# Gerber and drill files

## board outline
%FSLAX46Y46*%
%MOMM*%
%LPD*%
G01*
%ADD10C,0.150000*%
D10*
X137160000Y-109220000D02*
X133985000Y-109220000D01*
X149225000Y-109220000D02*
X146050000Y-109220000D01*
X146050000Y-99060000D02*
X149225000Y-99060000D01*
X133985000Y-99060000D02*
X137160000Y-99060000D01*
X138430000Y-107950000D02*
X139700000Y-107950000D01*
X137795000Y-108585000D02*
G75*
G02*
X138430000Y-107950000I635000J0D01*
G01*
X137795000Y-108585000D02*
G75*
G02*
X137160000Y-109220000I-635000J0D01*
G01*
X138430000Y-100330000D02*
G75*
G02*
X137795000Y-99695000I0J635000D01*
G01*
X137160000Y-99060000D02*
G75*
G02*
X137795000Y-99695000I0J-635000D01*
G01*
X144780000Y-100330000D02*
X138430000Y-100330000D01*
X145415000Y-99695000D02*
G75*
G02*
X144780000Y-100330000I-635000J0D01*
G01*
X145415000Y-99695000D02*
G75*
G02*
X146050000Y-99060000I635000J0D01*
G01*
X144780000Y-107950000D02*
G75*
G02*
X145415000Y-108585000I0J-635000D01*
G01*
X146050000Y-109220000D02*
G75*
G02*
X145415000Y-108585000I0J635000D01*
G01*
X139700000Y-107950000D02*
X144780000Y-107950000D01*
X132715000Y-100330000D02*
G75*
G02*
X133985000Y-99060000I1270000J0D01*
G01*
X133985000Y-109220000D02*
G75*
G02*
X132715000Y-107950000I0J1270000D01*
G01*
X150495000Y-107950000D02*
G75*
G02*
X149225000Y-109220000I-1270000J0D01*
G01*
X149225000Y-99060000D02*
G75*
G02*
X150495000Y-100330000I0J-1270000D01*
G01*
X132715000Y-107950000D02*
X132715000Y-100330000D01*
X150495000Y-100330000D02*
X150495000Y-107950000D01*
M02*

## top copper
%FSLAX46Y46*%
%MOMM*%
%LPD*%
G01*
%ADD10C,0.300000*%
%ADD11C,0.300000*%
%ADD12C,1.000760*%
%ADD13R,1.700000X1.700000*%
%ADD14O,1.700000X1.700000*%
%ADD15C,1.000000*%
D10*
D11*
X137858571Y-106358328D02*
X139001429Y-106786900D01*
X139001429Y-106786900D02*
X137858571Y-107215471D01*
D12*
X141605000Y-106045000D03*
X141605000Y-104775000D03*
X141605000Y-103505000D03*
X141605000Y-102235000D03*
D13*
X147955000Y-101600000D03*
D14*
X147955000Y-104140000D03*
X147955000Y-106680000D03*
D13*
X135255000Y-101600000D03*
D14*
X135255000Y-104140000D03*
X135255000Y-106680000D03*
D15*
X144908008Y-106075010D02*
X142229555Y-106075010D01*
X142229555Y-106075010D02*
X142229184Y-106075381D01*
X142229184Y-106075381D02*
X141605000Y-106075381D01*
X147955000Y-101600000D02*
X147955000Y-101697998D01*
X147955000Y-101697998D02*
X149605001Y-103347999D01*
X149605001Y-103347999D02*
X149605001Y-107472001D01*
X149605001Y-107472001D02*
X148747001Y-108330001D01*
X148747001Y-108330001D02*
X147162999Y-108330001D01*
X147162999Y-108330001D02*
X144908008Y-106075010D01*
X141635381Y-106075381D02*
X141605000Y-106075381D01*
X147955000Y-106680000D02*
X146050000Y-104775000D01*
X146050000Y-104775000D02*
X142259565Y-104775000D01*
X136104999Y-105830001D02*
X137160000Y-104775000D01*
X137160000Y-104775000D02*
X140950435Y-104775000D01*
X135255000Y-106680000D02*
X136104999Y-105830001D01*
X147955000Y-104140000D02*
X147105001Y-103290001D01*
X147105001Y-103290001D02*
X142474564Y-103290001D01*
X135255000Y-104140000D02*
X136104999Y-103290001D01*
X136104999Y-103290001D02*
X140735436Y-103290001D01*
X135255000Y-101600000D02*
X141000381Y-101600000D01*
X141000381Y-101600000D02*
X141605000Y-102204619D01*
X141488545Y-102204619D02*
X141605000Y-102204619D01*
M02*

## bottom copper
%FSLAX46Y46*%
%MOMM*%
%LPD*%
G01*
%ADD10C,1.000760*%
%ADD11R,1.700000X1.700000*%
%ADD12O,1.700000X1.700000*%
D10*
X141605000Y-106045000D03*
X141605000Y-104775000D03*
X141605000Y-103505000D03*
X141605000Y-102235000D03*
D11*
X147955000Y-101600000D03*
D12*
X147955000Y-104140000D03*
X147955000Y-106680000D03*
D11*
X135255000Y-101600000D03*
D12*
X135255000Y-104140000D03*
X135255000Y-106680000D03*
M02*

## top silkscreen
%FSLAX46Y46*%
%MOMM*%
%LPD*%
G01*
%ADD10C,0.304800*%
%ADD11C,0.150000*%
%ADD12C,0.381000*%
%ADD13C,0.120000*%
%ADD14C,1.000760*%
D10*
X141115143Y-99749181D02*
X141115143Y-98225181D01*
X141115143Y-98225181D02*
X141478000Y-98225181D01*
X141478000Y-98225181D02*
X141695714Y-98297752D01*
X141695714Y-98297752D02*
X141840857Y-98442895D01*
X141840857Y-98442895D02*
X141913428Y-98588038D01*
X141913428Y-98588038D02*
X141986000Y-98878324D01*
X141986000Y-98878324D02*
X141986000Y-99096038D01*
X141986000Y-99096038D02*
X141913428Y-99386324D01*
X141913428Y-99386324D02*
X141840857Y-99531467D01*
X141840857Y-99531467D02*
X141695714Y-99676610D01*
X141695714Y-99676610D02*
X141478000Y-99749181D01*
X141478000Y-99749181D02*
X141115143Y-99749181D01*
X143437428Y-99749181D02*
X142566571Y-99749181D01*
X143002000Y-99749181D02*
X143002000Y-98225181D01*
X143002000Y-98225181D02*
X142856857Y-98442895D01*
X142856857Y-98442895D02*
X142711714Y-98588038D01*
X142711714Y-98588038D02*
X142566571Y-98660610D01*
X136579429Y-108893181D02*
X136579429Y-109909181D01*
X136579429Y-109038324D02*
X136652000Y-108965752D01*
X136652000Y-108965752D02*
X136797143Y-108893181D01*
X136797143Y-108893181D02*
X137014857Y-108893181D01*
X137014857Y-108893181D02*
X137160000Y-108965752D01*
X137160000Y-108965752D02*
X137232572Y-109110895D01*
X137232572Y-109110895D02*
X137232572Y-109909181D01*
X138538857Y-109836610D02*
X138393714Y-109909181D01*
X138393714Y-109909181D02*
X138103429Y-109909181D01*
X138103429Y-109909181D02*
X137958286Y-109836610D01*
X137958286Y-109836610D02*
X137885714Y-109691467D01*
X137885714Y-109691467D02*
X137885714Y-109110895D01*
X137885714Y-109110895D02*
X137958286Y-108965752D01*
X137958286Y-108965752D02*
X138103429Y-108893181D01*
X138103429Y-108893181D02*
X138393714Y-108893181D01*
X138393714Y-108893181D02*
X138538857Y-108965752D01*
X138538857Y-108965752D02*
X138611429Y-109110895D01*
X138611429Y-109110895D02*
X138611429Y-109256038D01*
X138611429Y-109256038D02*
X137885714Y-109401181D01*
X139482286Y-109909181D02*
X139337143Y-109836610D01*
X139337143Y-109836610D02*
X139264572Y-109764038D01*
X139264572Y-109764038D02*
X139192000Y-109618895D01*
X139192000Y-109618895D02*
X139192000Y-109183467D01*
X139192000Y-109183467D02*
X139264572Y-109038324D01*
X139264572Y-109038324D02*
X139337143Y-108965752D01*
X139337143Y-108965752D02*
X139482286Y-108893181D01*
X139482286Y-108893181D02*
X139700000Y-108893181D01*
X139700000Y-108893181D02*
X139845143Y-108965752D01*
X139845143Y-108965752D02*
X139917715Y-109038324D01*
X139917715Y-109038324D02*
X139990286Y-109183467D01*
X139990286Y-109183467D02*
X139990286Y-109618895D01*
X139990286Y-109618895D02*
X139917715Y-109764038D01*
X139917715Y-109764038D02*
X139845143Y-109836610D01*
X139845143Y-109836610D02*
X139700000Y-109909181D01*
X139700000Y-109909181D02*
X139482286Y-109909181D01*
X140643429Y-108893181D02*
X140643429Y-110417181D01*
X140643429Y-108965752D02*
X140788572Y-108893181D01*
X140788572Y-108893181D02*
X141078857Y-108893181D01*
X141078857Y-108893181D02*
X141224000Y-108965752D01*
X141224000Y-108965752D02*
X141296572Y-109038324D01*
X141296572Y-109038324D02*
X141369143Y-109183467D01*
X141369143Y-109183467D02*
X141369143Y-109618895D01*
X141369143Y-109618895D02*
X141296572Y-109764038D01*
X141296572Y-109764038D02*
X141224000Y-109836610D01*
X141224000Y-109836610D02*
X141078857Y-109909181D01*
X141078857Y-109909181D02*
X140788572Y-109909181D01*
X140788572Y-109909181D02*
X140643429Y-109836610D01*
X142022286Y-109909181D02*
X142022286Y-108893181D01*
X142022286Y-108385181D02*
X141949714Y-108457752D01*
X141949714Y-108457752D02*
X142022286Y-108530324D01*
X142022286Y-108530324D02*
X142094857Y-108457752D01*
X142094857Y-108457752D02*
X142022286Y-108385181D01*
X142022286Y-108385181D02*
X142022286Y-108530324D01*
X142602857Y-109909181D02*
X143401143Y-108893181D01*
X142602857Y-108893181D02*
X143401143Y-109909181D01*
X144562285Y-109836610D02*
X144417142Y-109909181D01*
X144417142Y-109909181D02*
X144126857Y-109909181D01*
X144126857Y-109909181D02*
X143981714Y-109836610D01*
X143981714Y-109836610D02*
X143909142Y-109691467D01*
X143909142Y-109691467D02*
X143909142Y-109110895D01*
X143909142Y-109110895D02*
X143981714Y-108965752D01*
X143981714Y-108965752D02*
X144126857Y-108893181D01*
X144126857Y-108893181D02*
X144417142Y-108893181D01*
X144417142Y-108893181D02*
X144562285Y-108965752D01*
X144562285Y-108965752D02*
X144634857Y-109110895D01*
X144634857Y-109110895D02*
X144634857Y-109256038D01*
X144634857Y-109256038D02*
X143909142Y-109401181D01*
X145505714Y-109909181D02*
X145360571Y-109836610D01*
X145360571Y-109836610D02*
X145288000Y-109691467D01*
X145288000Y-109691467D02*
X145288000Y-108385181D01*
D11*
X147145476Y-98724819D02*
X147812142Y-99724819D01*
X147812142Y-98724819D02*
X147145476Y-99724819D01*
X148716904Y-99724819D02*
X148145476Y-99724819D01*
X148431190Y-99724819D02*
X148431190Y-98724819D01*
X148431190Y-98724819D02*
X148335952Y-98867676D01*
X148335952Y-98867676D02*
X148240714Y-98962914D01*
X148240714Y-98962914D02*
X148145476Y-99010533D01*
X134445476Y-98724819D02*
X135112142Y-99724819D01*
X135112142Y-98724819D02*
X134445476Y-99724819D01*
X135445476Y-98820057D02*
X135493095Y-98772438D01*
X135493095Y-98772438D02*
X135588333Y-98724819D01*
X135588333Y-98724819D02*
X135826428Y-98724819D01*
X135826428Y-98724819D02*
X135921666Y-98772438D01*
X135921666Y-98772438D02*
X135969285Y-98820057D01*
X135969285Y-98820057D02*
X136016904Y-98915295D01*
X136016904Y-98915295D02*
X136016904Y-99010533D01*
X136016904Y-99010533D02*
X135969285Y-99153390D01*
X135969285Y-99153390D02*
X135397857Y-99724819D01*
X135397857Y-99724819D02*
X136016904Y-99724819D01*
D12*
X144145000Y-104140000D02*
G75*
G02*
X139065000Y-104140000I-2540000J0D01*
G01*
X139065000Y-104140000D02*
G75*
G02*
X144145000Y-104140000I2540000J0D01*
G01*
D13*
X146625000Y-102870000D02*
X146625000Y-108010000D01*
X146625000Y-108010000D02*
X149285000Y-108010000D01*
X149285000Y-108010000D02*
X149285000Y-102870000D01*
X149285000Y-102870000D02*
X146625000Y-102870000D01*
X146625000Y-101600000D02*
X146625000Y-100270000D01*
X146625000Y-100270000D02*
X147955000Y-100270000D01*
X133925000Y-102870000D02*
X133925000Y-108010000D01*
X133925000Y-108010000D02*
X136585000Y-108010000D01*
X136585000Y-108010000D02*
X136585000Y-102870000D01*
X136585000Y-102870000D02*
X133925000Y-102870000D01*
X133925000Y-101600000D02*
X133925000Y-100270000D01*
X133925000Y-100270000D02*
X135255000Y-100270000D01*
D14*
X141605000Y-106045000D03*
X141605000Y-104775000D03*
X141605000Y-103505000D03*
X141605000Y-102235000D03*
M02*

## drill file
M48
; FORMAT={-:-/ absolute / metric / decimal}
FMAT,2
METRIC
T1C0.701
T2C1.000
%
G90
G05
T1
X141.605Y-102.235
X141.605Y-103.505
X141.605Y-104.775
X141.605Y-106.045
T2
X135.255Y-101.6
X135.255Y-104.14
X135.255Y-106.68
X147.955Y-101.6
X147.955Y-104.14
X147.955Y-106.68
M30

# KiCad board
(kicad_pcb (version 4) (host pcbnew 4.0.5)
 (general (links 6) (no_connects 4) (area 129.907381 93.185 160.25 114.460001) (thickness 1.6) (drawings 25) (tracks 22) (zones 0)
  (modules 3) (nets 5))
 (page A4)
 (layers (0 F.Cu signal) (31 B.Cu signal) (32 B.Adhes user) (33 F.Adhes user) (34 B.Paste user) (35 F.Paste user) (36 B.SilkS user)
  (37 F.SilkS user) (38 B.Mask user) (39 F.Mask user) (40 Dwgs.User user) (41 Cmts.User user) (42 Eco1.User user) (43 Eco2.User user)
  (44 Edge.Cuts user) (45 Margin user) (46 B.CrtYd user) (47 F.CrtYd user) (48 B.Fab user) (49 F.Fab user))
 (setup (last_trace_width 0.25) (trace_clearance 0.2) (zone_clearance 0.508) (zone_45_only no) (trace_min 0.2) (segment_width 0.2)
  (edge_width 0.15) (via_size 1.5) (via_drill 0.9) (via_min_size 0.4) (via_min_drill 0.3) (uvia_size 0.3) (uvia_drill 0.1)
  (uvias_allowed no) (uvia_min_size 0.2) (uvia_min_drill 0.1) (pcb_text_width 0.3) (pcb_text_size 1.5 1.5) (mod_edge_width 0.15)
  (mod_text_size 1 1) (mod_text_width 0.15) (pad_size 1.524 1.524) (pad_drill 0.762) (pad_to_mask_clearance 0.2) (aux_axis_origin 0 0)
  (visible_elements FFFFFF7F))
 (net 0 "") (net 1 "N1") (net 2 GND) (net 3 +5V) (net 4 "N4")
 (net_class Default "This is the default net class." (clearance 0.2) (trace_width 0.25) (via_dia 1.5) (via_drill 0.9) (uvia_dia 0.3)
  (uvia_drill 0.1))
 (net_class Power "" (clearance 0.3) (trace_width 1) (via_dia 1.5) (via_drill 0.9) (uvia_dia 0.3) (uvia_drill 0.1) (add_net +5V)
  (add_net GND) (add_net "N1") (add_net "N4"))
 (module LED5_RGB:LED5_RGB (layer F.Cu) (at 141.605 104.14 90)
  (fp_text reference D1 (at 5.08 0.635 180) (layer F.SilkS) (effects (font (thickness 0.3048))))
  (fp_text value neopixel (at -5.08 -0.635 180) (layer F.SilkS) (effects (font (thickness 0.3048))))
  (fp_circle (center 0 0) (end 2.54 0) (layer F.SilkS) (width 0.381))
  (pad 1 thru_hole circle (at -1.905 0 90) (size 1.00076 1.00076) (drill 0.70104) (layers *.Cu *.Mask F.SilkS) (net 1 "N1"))
  (pad 2 thru_hole circle (at -0.635 0 90) (size 1.00076 1.00076) (drill 0.70104) (layers *.Cu *.Mask F.SilkS) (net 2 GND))
  (pad 3 thru_hole circle (at 0.635 0 90) (size 1.00076 1.00076) (drill 0.70104) (layers *.Cu *.Mask F.SilkS) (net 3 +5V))
  (pad 4 thru_hole circle (at 1.905 0 90) (size 1.00076 1.00076) (drill 0.70104) (layers *.Cu *.Mask F.SilkS) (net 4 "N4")))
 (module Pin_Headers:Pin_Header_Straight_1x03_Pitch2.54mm (layer F.Cu) (at 147.955 101.6)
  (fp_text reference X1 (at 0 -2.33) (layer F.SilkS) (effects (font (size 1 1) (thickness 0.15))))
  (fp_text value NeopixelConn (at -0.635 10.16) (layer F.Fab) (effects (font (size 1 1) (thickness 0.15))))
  (fp_line (start -1.33 1.27) (end -1.33 6.41) (layer F.SilkS) (width 0.12))
  (fp_line (start -1.33 6.41) (end 1.33 6.41) (layer F.SilkS) (width 0.12))
  (fp_line (start 1.33 6.41) (end 1.33 1.27) (layer F.SilkS) (width 0.12))
  (fp_line (start 1.33 1.27) (end -1.33 1.27) (layer F.SilkS) (width 0.12))
  (fp_line (start -1.33 0) (end -1.33 -1.33) (layer F.SilkS) (width 0.12))
  (fp_line (start -1.33 -1.33) (end 0 -1.33) (layer F.SilkS) (width 0.12))
  (pad 1 thru_hole rect (at 0 0) (size 1.7 1.7) (drill 1) (layers *.Cu *.Mask) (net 1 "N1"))
  (pad 2 thru_hole oval (at 0 2.54) (size 1.7 1.7) (drill 1) (layers *.Cu *.Mask) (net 3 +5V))
  (pad 3 thru_hole oval (at 0 5.08) (size 1.7 1.7) (drill 1) (layers *.Cu *.Mask) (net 2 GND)))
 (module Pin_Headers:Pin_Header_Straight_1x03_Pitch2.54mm (layer F.Cu) (at 135.255 101.6)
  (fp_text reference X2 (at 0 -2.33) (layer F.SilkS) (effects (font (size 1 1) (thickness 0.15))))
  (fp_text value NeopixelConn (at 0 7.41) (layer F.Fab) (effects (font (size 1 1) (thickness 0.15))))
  (fp_line (start -1.33 1.27) (end -1.33 6.41) (layer F.SilkS) (width 0.12))
  (fp_line (start -1.33 6.41) (end 1.33 6.41) (layer F.SilkS) (width 0.12))
  (fp_line (start 1.33 6.41) (end 1.33 1.27) (layer F.SilkS) (width 0.12))
  (fp_line (start 1.33 1.27) (end -1.33 1.27) (layer F.SilkS) (width 0.12))
  (fp_line (start -1.33 0) (end -1.33 -1.33) (layer F.SilkS) (width 0.12))
  (fp_line (start -1.33 -1.33) (end 0 -1.33) (layer F.SilkS) (width 0.12))
  (pad 1 thru_hole rect (at 0 0) (size 1.7 1.7) (drill 1) (layers *.Cu *.Mask) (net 4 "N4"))
  (pad 2 thru_hole oval (at 0 2.54) (size 1.7 1.7) (drill 1) (layers *.Cu *.Mask) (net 3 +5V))
  (pad 3 thru_hole oval (at 0 5.08) (size 1.7 1.7) (drill 1) (layers *.Cu *.Mask) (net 2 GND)))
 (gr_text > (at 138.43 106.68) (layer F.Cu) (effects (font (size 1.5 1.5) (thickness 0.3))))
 (gr_line (start 137.16 109.22) (end 133.985 109.22) (layer Edge.Cuts) (width 0.15))
 (gr_line (start 149.225 109.22) (end 146.05 109.22) (layer Edge.Cuts) (width 0.15))
 (gr_line (start 146.05 99.06) (end 149.225 99.06) (layer Edge.Cuts) (width 0.15))
 (gr_line (start 133.985 99.06) (end 137.16 99.06) (layer Edge.Cuts) (width 0.15))
 (gr_line (start 138.43 107.95) (end 139.7 107.95) (layer Edge.Cuts) (width 0.15))
 (gr_arc (start 138.43 108.585) (end 137.795 108.585) (angle 90) (layer Edge.Cuts) (width 0.15))
 (gr_arc (start 137.16 108.585) (end 137.795 108.585) (angle 90) (layer Edge.Cuts) (width 0.15))
 (gr_arc (start 138.43 99.695) (end 138.43 100.33) (angle 90) (layer Edge.Cuts) (width 0.15))
 (gr_arc (start 137.16 99.695) (end 137.16 99.06) (angle 90) (layer Edge.Cuts) (width 0.15))
 (gr_line (start 144.78 100.33) (end 138.43 100.33) (layer Edge.Cuts) (width 0.15))
 (gr_arc (start 144.78 99.695) (end 145.415 99.695) (angle 90) (layer Edge.Cuts) (width 0.15))
 (gr_arc (start 146.05 99.695) (end 145.415 99.695) (angle 90) (layer Edge.Cuts) (width 0.15))
 (gr_arc (start 144.78 108.585) (end 144.78 107.95) (angle 90) (layer Edge.Cuts) (width 0.15))
 (gr_arc (start 146.05 108.585) (end 146.05 109.22) (angle 90) (layer Edge.Cuts) (width 0.15))
 (gr_line (start 139.7 107.95) (end 144.78 107.95) (layer Edge.Cuts) (width 0.15))
 (gr_arc (start 133.985 100.33) (end 132.715 100.33) (angle 90) (layer Edge.Cuts) (width 0.15))
 (gr_arc (start 133.985 107.95) (end 133.985 109.22) (angle 90) (layer Edge.Cuts) (width 0.15))
 (gr_arc (start 149.225 107.95) (end 150.495 107.95) (angle 90) (layer Edge.Cuts) (width 0.15))
 (gr_arc (start 149.225 100.33) (end 149.225 99.06) (angle 90) (layer Edge.Cuts) (width 0.15))
 (gr_line (start 132.715 107.95) (end 132.715 100.33) (layer Edge.Cuts) (width 0.15))
 (gr_line (start 150.495 100.33) (end 150.495 107.95) (layer Edge.Cuts) (width 0.15))
 (segment (start 144.908008 106.07501) (end 142.229555 106.07501) (width 1) (layer F.Cu) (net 1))
 (segment (start 142.229555 106.07501) (end 142.229184 106.075381) (width 1) (layer F.Cu) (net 1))
 (segment (start 142.229184 106.075381) (end 141.605 106.075381) (width 1) (layer F.Cu) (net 1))
 (segment (start 147.955 101.6) (end 147.955 101.697998) (width 1) (layer F.Cu) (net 1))
 (segment (start 147.955 101.697998) (end 149.605001 103.347999) (width 1) (layer F.Cu) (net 1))
 (segment (start 149.605001 103.347999) (end 149.605001 107.472001) (width 1) (layer F.Cu) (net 1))
 (segment (start 149.605001 107.472001) (end 148.747001 108.330001) (width 1) (layer F.Cu) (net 1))
 (segment (start 148.747001 108.330001) (end 147.162999 108.330001) (width 1) (layer F.Cu) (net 1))
 (segment (start 147.162999 108.330001) (end 144.908008 106.07501) (width 1) (layer F.Cu) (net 1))
 (segment (start 141.635381 106.075381) (end 141.605 106.075381) (width 1) (layer F.Cu) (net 1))
 (segment (start 147.955 106.68) (end 146.05 104.775) (width 1) (layer F.Cu) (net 2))
 (segment (start 146.05 104.775) (end 142.259565 104.775) (width 1) (layer F.Cu) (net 2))
 (segment (start 136.104999 105.830001) (end 137.16 104.775) (width 1) (layer F.Cu) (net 2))
 (segment (start 137.16 104.775) (end 140.950435 104.775) (width 1) (layer F.Cu) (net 2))
 (segment (start 135.255 106.68) (end 136.104999 105.830001) (width 1) (layer F.Cu) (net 2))
 (segment (start 147.955 104.14) (end 147.105001 103.290001) (width 1) (layer F.Cu) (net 3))
 (segment (start 147.105001 103.290001) (end 142.474564 103.290001) (width 1) (layer F.Cu) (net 3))
 (segment (start 135.255 104.14) (end 136.104999 103.290001) (width 1) (layer F.Cu) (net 3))
 (segment (start 136.104999 103.290001) (end 140.735436 103.290001) (width 1) (layer F.Cu) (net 3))
 (segment (start 135.255 101.6) (end 141.000381 101.6) (width 1) (layer F.Cu) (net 4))
 (segment (start 141.000381 101.6) (end 141.605 102.204619) (width 1) (layer F.Cu) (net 4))
 (segment (start 141.488545 102.204619) (end 141.605 102.204619) (width 1) (layer F.Cu) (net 4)))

